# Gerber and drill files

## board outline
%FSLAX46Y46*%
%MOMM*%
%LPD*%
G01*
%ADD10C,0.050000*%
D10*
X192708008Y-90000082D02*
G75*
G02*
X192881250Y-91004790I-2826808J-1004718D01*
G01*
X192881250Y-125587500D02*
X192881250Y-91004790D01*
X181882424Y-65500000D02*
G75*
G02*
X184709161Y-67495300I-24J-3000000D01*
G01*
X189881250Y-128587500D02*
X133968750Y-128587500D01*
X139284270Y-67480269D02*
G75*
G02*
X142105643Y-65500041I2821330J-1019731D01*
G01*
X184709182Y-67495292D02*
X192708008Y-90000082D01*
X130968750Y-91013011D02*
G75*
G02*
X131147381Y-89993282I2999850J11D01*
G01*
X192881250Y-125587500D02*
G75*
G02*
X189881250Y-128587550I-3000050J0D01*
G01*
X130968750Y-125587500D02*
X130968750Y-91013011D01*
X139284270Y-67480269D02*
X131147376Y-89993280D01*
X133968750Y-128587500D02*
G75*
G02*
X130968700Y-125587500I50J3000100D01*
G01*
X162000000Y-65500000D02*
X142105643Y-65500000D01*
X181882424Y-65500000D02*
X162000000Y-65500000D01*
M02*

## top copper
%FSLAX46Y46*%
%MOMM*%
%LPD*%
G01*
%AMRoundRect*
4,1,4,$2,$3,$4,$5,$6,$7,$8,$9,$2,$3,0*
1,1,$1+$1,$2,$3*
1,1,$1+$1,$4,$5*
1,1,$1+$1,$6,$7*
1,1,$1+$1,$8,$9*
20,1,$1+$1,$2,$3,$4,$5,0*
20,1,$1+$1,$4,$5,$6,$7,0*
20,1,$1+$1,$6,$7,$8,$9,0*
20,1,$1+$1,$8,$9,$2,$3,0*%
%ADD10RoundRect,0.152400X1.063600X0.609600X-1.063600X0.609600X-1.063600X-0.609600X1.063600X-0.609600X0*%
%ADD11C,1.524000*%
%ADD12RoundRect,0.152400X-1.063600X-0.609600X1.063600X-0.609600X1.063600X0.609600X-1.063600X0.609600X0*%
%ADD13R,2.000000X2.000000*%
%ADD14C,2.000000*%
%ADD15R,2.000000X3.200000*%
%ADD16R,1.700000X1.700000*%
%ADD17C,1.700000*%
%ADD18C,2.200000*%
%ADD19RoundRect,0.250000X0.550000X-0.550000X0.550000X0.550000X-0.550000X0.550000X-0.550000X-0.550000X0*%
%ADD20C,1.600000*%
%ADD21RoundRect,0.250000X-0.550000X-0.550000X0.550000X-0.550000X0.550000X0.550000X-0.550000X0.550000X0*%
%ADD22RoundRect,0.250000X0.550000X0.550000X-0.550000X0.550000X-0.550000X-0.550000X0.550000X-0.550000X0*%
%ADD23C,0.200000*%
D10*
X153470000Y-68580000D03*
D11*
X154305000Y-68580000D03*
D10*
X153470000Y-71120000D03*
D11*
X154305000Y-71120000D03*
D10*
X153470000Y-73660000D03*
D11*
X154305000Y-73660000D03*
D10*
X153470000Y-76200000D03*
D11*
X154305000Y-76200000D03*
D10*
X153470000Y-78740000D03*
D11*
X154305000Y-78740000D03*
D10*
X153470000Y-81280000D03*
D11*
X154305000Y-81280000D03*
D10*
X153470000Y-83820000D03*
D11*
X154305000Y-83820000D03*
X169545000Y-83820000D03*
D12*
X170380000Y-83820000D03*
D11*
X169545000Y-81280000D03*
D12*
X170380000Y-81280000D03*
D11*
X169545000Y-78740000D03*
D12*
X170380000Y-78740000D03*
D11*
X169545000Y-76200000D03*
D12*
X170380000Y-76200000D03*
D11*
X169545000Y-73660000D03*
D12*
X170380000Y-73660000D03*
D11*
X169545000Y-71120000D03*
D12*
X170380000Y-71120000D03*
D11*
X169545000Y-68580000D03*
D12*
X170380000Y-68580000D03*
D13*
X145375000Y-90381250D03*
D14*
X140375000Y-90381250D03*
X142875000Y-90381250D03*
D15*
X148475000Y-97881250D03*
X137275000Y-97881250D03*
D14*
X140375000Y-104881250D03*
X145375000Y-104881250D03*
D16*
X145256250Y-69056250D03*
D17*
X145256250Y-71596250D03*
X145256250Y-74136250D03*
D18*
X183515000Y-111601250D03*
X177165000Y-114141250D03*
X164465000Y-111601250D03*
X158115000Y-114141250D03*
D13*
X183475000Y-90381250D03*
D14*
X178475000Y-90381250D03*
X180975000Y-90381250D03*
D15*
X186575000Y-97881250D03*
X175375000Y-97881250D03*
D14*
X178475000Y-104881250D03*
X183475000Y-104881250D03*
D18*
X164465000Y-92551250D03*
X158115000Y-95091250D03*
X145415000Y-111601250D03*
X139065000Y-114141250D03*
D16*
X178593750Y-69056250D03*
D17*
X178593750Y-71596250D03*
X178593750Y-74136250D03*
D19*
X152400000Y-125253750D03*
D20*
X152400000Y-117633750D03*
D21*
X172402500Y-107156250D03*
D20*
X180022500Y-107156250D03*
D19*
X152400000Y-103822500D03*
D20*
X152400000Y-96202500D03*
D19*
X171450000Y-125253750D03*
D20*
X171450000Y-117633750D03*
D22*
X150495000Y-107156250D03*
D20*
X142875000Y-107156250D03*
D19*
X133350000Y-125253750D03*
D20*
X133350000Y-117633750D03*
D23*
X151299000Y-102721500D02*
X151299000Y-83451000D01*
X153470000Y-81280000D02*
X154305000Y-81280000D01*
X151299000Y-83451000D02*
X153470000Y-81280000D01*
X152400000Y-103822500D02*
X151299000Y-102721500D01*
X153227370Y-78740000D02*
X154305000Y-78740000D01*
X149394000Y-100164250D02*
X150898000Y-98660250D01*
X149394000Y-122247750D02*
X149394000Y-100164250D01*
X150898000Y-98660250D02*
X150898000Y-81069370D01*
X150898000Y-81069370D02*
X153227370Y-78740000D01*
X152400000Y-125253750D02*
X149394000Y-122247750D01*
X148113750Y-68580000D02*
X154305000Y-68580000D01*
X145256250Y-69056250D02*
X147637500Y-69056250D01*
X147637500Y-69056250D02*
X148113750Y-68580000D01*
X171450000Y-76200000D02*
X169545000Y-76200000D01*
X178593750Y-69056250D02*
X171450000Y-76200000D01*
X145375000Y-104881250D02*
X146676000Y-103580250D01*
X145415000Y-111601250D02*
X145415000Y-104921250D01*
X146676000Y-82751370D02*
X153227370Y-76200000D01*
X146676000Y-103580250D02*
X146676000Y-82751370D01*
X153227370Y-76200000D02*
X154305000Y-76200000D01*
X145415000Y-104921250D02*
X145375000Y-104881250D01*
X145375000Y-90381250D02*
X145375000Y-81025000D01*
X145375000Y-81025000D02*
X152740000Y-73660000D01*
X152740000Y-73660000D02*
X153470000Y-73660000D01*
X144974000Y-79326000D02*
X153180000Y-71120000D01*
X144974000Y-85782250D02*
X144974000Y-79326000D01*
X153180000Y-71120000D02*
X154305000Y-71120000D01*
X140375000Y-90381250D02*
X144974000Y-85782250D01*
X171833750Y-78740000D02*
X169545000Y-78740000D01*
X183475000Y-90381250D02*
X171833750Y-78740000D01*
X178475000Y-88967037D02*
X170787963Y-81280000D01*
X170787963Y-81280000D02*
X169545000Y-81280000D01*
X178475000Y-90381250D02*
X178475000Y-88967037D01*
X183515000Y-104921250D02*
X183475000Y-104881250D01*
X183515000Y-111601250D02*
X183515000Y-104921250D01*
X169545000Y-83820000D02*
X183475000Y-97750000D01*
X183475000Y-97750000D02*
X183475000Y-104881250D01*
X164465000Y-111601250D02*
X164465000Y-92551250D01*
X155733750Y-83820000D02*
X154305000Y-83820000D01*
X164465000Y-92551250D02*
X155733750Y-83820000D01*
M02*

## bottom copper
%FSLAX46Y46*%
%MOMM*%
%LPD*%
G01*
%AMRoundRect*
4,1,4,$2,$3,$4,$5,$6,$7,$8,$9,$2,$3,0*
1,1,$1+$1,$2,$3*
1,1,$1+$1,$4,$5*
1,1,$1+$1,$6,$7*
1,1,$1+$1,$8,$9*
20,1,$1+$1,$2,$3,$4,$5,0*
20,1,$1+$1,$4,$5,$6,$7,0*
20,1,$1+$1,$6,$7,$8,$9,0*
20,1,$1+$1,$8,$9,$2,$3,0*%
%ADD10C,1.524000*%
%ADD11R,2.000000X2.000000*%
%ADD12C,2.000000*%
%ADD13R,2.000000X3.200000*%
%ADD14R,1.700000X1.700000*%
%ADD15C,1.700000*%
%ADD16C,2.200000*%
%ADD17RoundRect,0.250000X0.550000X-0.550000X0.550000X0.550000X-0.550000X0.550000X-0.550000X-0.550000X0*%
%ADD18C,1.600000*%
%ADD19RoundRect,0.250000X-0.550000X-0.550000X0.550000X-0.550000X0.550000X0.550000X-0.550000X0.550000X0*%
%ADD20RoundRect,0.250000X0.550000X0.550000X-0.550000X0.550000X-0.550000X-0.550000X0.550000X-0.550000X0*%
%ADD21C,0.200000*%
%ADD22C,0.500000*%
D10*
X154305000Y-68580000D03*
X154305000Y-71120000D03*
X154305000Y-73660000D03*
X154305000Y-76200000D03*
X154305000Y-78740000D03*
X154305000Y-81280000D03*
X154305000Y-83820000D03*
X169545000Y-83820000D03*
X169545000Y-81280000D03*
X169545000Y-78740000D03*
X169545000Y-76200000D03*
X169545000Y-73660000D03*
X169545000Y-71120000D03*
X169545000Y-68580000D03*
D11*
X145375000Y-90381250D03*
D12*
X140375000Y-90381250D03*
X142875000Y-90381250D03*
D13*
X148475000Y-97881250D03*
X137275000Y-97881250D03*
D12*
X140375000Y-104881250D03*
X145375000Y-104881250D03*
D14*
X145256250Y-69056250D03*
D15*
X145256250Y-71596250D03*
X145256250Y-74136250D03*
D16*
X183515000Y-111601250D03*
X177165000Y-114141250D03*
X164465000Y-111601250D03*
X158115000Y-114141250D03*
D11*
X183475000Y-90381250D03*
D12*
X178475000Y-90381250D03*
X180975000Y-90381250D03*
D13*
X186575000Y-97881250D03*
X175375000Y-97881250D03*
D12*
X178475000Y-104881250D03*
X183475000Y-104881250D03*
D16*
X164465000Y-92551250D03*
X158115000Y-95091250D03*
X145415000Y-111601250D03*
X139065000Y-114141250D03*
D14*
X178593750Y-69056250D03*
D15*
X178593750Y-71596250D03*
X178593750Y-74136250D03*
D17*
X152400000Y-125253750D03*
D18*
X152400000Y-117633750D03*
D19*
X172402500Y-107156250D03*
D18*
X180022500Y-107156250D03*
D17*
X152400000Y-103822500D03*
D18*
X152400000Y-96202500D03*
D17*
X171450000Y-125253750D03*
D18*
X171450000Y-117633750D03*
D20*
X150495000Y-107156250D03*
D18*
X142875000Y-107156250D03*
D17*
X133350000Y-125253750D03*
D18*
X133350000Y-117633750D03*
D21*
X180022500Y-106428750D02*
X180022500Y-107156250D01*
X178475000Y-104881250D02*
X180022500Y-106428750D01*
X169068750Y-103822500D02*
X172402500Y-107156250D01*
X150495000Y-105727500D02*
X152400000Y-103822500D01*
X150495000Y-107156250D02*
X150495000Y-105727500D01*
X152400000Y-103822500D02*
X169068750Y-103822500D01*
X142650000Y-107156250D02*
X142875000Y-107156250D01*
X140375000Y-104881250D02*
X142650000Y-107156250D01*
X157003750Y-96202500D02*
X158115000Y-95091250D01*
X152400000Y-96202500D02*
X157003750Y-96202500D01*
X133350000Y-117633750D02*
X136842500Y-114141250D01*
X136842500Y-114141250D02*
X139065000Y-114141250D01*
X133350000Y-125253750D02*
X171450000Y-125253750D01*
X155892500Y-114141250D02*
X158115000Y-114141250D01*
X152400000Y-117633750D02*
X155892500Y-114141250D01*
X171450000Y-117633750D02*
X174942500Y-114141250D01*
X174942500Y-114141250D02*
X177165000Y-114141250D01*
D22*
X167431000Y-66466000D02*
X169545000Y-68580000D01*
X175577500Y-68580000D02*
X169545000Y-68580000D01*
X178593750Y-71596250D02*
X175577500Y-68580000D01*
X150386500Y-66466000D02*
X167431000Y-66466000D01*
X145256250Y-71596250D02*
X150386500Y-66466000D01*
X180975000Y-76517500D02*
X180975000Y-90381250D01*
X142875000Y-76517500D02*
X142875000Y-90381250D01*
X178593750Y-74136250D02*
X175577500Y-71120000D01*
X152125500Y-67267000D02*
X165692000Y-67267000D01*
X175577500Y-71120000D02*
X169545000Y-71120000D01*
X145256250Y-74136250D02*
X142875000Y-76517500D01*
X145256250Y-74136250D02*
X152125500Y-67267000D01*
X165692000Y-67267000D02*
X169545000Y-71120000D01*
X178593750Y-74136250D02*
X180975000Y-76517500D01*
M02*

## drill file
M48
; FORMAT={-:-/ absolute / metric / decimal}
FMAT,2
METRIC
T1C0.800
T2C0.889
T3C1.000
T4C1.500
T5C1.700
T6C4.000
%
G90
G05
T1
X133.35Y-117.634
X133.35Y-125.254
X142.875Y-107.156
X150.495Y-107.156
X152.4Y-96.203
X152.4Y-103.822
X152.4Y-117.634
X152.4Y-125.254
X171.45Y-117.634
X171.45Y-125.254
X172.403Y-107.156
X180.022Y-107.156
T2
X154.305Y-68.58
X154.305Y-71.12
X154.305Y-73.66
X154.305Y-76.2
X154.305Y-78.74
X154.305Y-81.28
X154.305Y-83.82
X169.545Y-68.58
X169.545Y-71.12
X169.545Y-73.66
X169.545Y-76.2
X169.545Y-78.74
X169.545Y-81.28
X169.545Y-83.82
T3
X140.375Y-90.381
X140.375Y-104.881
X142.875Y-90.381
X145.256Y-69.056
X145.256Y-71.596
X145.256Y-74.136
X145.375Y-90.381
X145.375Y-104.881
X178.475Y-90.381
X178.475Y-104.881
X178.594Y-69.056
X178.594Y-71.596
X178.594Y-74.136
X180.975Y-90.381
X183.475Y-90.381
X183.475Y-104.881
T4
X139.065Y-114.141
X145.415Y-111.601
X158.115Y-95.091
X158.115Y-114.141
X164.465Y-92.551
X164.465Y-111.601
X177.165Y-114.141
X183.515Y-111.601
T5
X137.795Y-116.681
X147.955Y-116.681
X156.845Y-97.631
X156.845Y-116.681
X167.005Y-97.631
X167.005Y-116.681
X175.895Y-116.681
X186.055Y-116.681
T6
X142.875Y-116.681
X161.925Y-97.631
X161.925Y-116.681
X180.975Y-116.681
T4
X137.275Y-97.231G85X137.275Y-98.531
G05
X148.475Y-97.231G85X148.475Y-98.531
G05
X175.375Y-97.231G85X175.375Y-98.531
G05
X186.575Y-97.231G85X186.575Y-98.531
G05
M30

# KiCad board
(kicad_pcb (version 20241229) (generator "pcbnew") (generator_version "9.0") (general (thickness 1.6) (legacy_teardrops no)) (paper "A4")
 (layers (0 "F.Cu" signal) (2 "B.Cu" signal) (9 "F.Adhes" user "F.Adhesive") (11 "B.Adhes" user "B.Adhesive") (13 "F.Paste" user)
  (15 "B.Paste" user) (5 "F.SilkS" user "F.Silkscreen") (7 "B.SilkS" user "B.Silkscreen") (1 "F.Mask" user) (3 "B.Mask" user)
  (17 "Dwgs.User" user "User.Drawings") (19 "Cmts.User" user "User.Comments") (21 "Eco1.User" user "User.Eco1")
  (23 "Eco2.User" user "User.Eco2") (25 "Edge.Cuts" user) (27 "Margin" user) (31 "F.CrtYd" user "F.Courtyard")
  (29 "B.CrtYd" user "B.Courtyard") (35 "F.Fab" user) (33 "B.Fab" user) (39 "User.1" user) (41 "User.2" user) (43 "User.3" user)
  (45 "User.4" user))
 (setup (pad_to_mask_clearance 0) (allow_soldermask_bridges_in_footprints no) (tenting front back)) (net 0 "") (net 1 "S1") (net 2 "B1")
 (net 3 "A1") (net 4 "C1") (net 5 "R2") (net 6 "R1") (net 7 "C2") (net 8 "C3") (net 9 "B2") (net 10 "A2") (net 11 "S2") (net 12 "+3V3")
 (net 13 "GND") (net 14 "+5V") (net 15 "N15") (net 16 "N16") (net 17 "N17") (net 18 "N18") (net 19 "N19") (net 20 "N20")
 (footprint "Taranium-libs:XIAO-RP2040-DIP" (layer "F.Cu") (at 161.925 76.2)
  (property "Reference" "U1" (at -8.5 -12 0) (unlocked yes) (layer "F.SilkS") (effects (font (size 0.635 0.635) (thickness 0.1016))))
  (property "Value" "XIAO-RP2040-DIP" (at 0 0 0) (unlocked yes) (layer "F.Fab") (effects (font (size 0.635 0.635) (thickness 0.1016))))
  (pad "1" smd roundrect (at -8.455 -7.62 180) (size 2.432 1.524) (layers "F.Cu" "F.Mask") (roundrect_rratio 0.1) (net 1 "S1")
   (thermal_bridge_angle 45))
  (pad "1" thru_hole circle (at -7.62 -7.62 180) (size 1.524 1.524) (drill 0.889) (layers "*.Cu" "*.Mask") (remove_unused_layers no)
   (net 1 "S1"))
  (pad "2" smd roundrect (at -8.455 -5.08 180) (size 2.432 1.524) (layers "F.Cu" "F.Mask") (roundrect_rratio 0.1) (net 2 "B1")
   (thermal_bridge_angle 45))
  (pad "2" thru_hole circle (at -7.62 -5.08 180) (size 1.524 1.524) (drill 0.889) (layers "*.Cu" "*.Mask") (remove_unused_layers no)
   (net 2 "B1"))
  (pad "3" smd roundrect (at -8.455 -2.54 180) (size 2.432 1.524) (layers "F.Cu" "F.Mask") (roundrect_rratio 0.1) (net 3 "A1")
   (thermal_bridge_angle 45))
  (pad "3" thru_hole circle (at -7.62 -2.54 180) (size 1.524 1.524) (drill 0.889) (layers "*.Cu" "*.Mask") (remove_unused_layers no)
   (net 3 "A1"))
  (pad "4" smd roundrect (at -8.455 0 180) (size 2.432 1.524) (layers "F.Cu" "F.Mask") (roundrect_rratio 0.1) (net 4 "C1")
   (thermal_bridge_angle 45))
  (pad "4" thru_hole circle (at -7.62 0 180) (size 1.524 1.524) (drill 0.889) (layers "*.Cu" "*.Mask") (remove_unused_layers no)
   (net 4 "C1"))
  (pad "5" smd roundrect (at -8.455 2.54 180) (size 2.432 1.524) (layers "F.Cu" "F.Mask") (roundrect_rratio 0.1) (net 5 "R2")
   (thermal_bridge_angle 45))
  (pad "5" thru_hole circle (at -7.62 2.54 180) (size 1.524 1.524) (drill 0.889) (layers "*.Cu" "*.Mask") (remove_unused_layers no)
   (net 5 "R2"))
  (pad "6" smd roundrect (at -8.455 5.08 180) (size 2.432 1.524) (layers "F.Cu" "F.Mask") (roundrect_rratio 0.1) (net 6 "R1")
   (thermal_bridge_angle 45))
  (pad "6" thru_hole circle (at -7.62 5.08 180) (size 1.524 1.524) (drill 0.889) (layers "*.Cu" "*.Mask") (remove_unused_layers no)
   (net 6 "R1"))
  (pad "7" smd roundrect (at -8.455 7.62 180) (size 2.432 1.524) (layers "F.Cu" "F.Mask") (roundrect_rratio 0.1) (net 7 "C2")
   (thermal_bridge_angle 45))
  (pad "7" thru_hole circle (at -7.62 7.62 180) (size 1.524 1.524) (drill 0.889) (layers "*.Cu" "*.Mask") (remove_unused_layers no)
   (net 7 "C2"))
  (pad "8" thru_hole circle (at 7.62 7.62) (size 1.524 1.524) (drill 0.889) (layers "*.Cu" "*.Mask") (remove_unused_layers no) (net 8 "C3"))
  (pad "8" smd roundrect (at 8.455 7.62) (size 2.432 1.524) (layers "F.Cu" "F.Mask") (roundrect_rratio 0.1) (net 8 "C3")
   (thermal_bridge_angle 45))
  (pad "9" thru_hole circle (at 7.62 5.08) (size 1.524 1.524) (drill 0.889) (layers "*.Cu" "*.Mask") (remove_unused_layers no) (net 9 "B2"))
  (pad "9" smd roundrect (at 8.455 5.08) (size 2.432 1.524) (layers "F.Cu" "F.Mask") (roundrect_rratio 0.1) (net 9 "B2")
   (thermal_bridge_angle 45))
  (pad "10" thru_hole circle (at 7.62 2.54) (size 1.524 1.524) (drill 0.889) (layers "*.Cu" "*.Mask") (remove_unused_layers no)
   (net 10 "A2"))
  (pad "10" smd roundrect (at 8.455 2.54) (size 2.432 1.524) (layers "F.Cu" "F.Mask") (roundrect_rratio 0.1) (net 10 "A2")
   (thermal_bridge_angle 45))
  (pad "11" thru_hole circle (at 7.62 0) (size 1.524 1.524) (drill 0.889) (layers "*.Cu" "*.Mask") (remove_unused_layers no) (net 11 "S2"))
  (pad "11" smd roundrect (at 8.455 0) (size 2.432 1.524) (layers "F.Cu" "F.Mask") (roundrect_rratio 0.1) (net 11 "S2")
   (thermal_bridge_angle 45))
  (pad "12" thru_hole circle (at 7.62 -2.54) (size 1.524 1.524) (drill 0.889) (layers "*.Cu" "*.Mask") (remove_unused_layers no)
   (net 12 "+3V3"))
  (pad "12" smd roundrect (at 8.455 -2.54) (size 2.432 1.524) (layers "F.Cu" "F.Mask") (roundrect_rratio 0.1) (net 12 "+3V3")
   (thermal_bridge_angle 45))
  (pad "13" thru_hole circle (at 7.62 -5.08) (size 1.524 1.524) (drill 0.889) (layers "*.Cu" "*.Mask") (remove_unused_layers no)
   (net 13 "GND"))
  (pad "13" smd roundrect (at 8.455 -5.08) (size 2.432 1.524) (layers "F.Cu" "F.Mask") (roundrect_rratio 0.1) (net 13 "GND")
   (thermal_bridge_angle 45))
  (pad "14" thru_hole circle (at 7.62 -7.62) (size 1.524 1.524) (drill 0.889) (layers "*.Cu" "*.Mask") (remove_unused_layers no)
   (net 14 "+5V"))
  (pad "14" smd roundrect (at 8.455 -7.62) (size 2.432 1.524) (layers "F.Cu" "F.Mask") (roundrect_rratio 0.1) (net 14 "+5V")
   (thermal_bridge_angle 45)))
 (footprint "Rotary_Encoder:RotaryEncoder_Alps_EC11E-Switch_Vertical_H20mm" (layer "F.Cu") (at 145.375 90.38125 -90)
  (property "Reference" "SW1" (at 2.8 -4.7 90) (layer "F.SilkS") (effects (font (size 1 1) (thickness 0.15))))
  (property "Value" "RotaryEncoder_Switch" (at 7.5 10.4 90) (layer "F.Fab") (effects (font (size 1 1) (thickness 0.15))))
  (pad "A" thru_hole rect (at 0 0 270) (size 2 2) (drill 1) (layers "*.Cu" "*.Mask") (remove_unused_layers no) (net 3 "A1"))
  (pad "B" thru_hole circle (at 0 5 270) (size 2 2) (drill 1) (layers "*.Cu" "*.Mask") (remove_unused_layers no) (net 2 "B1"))
  (pad "C" thru_hole circle (at 0 2.5 270) (size 2 2) (drill 1) (layers "*.Cu" "*.Mask") (remove_unused_layers no) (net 13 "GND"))
  (pad "MP" thru_hole rect (at 7.5 -3.1 270) (size 3.2 2) (drill oval 2.8 1.5) (layers "*.Cu" "*.Mask") (remove_unused_layers no))
  (pad "MP" thru_hole rect (at 7.5 8.1 270) (size 3.2 2) (drill oval 2.8 1.5) (layers "*.Cu" "*.Mask") (remove_unused_layers no))
  (pad "S1" thru_hole circle (at 14.5 5 270) (size 2 2) (drill 1) (layers "*.Cu" "*.Mask") (remove_unused_layers no) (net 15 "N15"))
  (pad "S2" thru_hole circle (at 14.5 0 270) (size 2 2) (drill 1) (layers "*.Cu" "*.Mask") (remove_unused_layers no) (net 4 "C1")))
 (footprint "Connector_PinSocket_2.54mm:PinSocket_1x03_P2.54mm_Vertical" (layer "F.Cu") (at 145.25625 69.05625)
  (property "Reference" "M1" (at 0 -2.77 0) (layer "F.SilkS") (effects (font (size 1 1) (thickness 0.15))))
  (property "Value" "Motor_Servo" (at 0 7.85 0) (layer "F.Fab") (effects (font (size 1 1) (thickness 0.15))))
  (pad "1" thru_hole rect (at 0 0) (size 1.7 1.7) (drill 1) (layers "*.Cu" "*.Mask") (remove_unused_layers no) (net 1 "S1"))
  (pad "2" thru_hole circle (at 0 2.54) (size 1.7 1.7) (drill 1) (layers "*.Cu" "*.Mask") (remove_unused_layers no) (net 14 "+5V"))
  (pad "3" thru_hole circle (at 0 5.08) (size 1.7 1.7) (drill 1) (layers "*.Cu" "*.Mask") (remove_unused_layers no) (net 13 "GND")))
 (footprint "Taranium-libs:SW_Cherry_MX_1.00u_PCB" (layer "F.Cu") (at 183.515 111.60125)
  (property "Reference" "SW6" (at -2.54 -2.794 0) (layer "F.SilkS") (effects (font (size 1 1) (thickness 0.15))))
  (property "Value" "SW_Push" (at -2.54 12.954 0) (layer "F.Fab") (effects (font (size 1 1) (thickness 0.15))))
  (pad "" np_thru_hole circle (at -7.62 5.08) (size 1.7 1.7) (drill 1.7) (layers "*.Cu" "*.Mask"))
  (pad "" np_thru_hole circle (at -2.54 5.08) (size 4 4) (drill 4) (layers "*.Cu" "*.Mask"))
  (pad "" np_thru_hole circle (at 2.54 5.08) (size 1.7 1.7) (drill 1.7) (layers "*.Cu" "*.Mask"))
  (pad "1" thru_hole circle (at 0 0) (size 2.2 2.2) (drill 1.5) (layers "*.Cu" "*.Mask") (remove_unused_layers no) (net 8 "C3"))
  (pad "2" thru_hole circle (at -6.35 2.54) (size 2.2 2.2) (drill 1.5) (layers "*.Cu" "*.Mask") (remove_unused_layers no) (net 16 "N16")))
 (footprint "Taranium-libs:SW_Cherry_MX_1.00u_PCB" (layer "F.Cu") (at 164.465 111.60125)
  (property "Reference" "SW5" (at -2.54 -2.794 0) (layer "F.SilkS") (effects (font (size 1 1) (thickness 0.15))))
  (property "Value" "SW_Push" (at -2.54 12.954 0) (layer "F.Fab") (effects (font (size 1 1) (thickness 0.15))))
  (pad "" np_thru_hole circle (at -7.62 5.08) (size 1.7 1.7) (drill 1.7) (layers "*.Cu" "*.Mask"))
  (pad "" np_thru_hole circle (at -2.54 5.08) (size 4 4) (drill 4) (layers "*.Cu" "*.Mask"))
  (pad "" np_thru_hole circle (at 2.54 5.08) (size 1.7 1.7) (drill 1.7) (layers "*.Cu" "*.Mask"))
  (pad "1" thru_hole circle (at 0 0) (size 2.2 2.2) (drill 1.5) (layers "*.Cu" "*.Mask") (remove_unused_layers no) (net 7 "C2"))
  (pad "2" thru_hole circle (at -6.35 2.54) (size 2.2 2.2) (drill 1.5) (layers "*.Cu" "*.Mask") (remove_unused_layers no) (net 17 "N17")))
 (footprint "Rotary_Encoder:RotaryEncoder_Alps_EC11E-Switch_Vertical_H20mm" (layer "F.Cu") (at 183.475 90.38125 -90)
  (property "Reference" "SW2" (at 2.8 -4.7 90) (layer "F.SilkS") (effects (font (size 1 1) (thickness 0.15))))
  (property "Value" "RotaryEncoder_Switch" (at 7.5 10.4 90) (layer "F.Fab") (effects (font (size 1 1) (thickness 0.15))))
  (pad "A" thru_hole rect (at 0 0 270) (size 2 2) (drill 1) (layers "*.Cu" "*.Mask") (remove_unused_layers no) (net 10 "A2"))
  (pad "B" thru_hole circle (at 0 5 270) (size 2 2) (drill 1) (layers "*.Cu" "*.Mask") (remove_unused_layers no) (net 9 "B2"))
  (pad "C" thru_hole circle (at 0 2.5 270) (size 2 2) (drill 1) (layers "*.Cu" "*.Mask") (remove_unused_layers no) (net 13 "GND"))
  (pad "MP" thru_hole rect (at 7.5 -3.1 270) (size 3.2 2) (drill oval 2.8 1.5) (layers "*.Cu" "*.Mask") (remove_unused_layers no))
  (pad "MP" thru_hole rect (at 7.5 8.1 270) (size 3.2 2) (drill oval 2.8 1.5) (layers "*.Cu" "*.Mask") (remove_unused_layers no))
  (pad "S1" thru_hole circle (at 14.5 5 270) (size 2 2) (drill 1) (layers "*.Cu" "*.Mask") (remove_unused_layers no) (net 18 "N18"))
  (pad "S2" thru_hole circle (at 14.5 0 270) (size 2 2) (drill 1) (layers "*.Cu" "*.Mask") (remove_unused_layers no) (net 8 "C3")))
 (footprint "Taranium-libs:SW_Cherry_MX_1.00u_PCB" (layer "F.Cu") (at 164.465 92.55125)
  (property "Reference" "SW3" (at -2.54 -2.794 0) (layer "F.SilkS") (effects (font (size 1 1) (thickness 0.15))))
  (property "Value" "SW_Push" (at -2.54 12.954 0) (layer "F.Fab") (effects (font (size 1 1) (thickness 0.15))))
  (pad "" np_thru_hole circle (at -7.62 5.08) (size 1.7 1.7) (drill 1.7) (layers "*.Cu" "*.Mask"))
  (pad "" np_thru_hole circle (at -2.54 5.08) (size 4 4) (drill 4) (layers "*.Cu" "*.Mask"))
  (pad "" np_thru_hole circle (at 2.54 5.08) (size 1.7 1.7) (drill 1.7) (layers "*.Cu" "*.Mask"))
  (pad "1" thru_hole circle (at 0 0) (size 2.2 2.2) (drill 1.5) (layers "*.Cu" "*.Mask") (remove_unused_layers no) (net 7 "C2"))
  (pad "2" thru_hole circle (at -6.35 2.54) (size 2.2 2.2) (drill 1.5) (layers "*.Cu" "*.Mask") (remove_unused_layers no) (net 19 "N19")))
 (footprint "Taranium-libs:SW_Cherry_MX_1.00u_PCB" (layer "F.Cu") (at 145.415 111.60125)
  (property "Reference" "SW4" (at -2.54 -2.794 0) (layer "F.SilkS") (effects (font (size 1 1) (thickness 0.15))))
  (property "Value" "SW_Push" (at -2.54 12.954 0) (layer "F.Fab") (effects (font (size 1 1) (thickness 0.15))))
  (pad "" np_thru_hole circle (at -7.62 5.08) (size 1.7 1.7) (drill 1.7) (layers "*.Cu" "*.Mask"))
  (pad "" np_thru_hole circle (at -2.54 5.08) (size 4 4) (drill 4) (layers "*.Cu" "*.Mask"))
  (pad "" np_thru_hole circle (at 2.54 5.08) (size 1.7 1.7) (drill 1.7) (layers "*.Cu" "*.Mask"))
  (pad "1" thru_hole circle (at 0 0) (size 2.2 2.2) (drill 1.5) (layers "*.Cu" "*.Mask") (remove_unused_layers no) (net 4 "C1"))
  (pad "2" thru_hole circle (at -6.35 2.54) (size 2.2 2.2) (drill 1.5) (layers "*.Cu" "*.Mask") (remove_unused_layers no) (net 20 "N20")))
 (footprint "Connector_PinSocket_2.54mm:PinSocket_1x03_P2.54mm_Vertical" (layer "F.Cu") (at 178.59375 69.05625)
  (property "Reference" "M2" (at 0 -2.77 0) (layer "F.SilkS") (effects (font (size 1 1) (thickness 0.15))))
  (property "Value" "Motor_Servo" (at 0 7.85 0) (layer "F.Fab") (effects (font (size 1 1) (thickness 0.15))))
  (pad "1" thru_hole rect (at 0 0) (size 1.7 1.7) (drill 1) (layers "*.Cu" "*.Mask") (remove_unused_layers no) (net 11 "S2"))
  (pad "2" thru_hole circle (at 0 2.54) (size 1.7 1.7) (drill 1) (layers "*.Cu" "*.Mask") (remove_unused_layers no) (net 14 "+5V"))
  (pad "3" thru_hole circle (at 0 5.08) (size 1.7 1.7) (drill 1) (layers "*.Cu" "*.Mask") (remove_unused_layers no) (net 13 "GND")))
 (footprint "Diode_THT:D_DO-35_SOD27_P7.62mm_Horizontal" (layer "B.Cu") (at 152.4 125.25375 90)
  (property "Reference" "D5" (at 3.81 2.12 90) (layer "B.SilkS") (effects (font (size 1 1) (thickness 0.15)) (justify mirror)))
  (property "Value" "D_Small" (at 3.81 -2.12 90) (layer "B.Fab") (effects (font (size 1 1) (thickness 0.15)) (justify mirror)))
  (pad "1" thru_hole roundrect (at 0 0 90) (size 1.6 1.6) (drill 0.8) (layers "*.Cu" "*.Mask") (remove_unused_layers no)
   (roundrect_rratio 0.15625) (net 5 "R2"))
  (pad "2" thru_hole circle (at 7.62 0 90) (size 1.6 1.6) (drill 0.8) (layers "*.Cu" "*.Mask") (remove_unused_layers no) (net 17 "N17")))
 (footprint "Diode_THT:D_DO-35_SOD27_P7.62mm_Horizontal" (layer "B.Cu") (at 172.4025 107.15625)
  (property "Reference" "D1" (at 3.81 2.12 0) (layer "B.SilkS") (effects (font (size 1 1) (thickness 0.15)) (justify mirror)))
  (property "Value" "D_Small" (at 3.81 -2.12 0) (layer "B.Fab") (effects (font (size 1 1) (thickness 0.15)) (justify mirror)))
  (pad "1" thru_hole roundrect (at 0 0) (size 1.6 1.6) (drill 0.8) (layers "*.Cu" "*.Mask") (remove_unused_layers no)
   (roundrect_rratio 0.15625) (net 6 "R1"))
  (pad "2" thru_hole circle (at 7.62 0) (size 1.6 1.6) (drill 0.8) (layers "*.Cu" "*.Mask") (remove_unused_layers no) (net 18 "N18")))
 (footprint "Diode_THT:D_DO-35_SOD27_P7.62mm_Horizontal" (layer "B.Cu") (at 152.4 103.8225 90)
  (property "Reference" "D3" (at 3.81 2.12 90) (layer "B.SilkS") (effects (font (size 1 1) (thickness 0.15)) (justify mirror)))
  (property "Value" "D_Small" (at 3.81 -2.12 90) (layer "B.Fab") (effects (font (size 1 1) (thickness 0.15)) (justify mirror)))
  (pad "1" thru_hole roundrect (at 0 0 90) (size 1.6 1.6) (drill 0.8) (layers "*.Cu" "*.Mask") (remove_unused_layers no)
   (roundrect_rratio 0.15625) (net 6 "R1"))
  (pad "2" thru_hole circle (at 7.62 0 90) (size 1.6 1.6) (drill 0.8) (layers "*.Cu" "*.Mask") (remove_unused_layers no) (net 19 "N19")))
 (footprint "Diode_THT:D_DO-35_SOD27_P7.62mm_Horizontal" (layer "B.Cu") (at 171.45 125.25375 90)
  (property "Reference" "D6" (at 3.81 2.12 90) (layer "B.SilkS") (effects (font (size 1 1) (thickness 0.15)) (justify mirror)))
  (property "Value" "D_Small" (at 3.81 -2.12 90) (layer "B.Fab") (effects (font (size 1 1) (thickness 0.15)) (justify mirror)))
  (pad "1" thru_hole roundrect (at 0 0 90) (size 1.6 1.6) (drill 0.8) (layers "*.Cu" "*.Mask") (remove_unused_layers no)
   (roundrect_rratio 0.15625) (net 5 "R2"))
  (pad "2" thru_hole circle (at 7.62 0 90) (size 1.6 1.6) (drill 0.8) (layers "*.Cu" "*.Mask") (remove_unused_layers no) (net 16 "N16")))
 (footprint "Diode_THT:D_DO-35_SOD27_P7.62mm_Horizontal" (layer "B.Cu") (at 150.495 107.15625 180)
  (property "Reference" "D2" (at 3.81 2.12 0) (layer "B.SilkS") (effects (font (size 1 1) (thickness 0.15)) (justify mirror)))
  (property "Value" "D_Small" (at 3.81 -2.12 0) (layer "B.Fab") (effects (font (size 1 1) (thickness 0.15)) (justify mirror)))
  (pad "1" thru_hole roundrect (at 0 0 180) (size 1.6 1.6) (drill 0.8) (layers "*.Cu" "*.Mask") (remove_unused_layers no)
   (roundrect_rratio 0.15625) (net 6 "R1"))
  (pad "2" thru_hole circle (at 7.62 0 180) (size 1.6 1.6) (drill 0.8) (layers "*.Cu" "*.Mask") (remove_unused_layers no) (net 15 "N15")))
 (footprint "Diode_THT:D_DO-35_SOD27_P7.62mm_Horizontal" (layer "B.Cu") (at 133.35 125.25375 90)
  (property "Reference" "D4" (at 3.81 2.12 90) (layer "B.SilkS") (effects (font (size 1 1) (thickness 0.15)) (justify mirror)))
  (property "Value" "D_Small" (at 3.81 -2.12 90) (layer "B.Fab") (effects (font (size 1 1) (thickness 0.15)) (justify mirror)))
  (pad "1" thru_hole roundrect (at 0 0 90) (size 1.6 1.6) (drill 0.8) (layers "*.Cu" "*.Mask") (remove_unused_layers no)
   (roundrect_rratio 0.15625) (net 5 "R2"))
  (pad "2" thru_hole circle (at 7.62 0 90) (size 1.6 1.6) (drill 0.8) (layers "*.Cu" "*.Mask") (remove_unused_layers no) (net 20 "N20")))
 (gr_arc (start 192.708008 90.000082) (mid 192.837622 90.495023) (end 192.88125 91.00479) (stroke (width 0.05) (type default))
  (layer "Edge.Cuts"))
 (gr_line (start 192.88125 125.5875) (end 192.88125 91.00479) (stroke (width 0.05) (type default)) (layer "Edge.Cuts"))
 (gr_arc (start 181.882424 65.5) (mid 183.612435 66.049069) (end 184.709182 67.495292) (stroke (width 0.05) (type default))
  (layer "Edge.Cuts"))
 (gr_line (start 189.88125 128.5875) (end 133.96875 128.5875) (stroke (width 0.05) (type default)) (layer "Edge.Cuts"))
 (gr_arc (start 139.28427 67.480269) (mid 140.382158 66.044477) (end 142.105643 65.5) (stroke (width 0.05) (type default))
  (layer "Edge.Cuts"))
 (gr_line (start 184.709182 67.495292) (end 192.708008 90.000082) (stroke (width 0.05) (type default)) (layer "Edge.Cuts"))
 (gr_arc (start 130.96875 91.013011) (mid 131.013741 90.495381) (end 131.147376 89.99328) (stroke (width 0.05) (type default))
  (layer "Edge.Cuts"))
 (gr_arc (start 192.88125 125.5875) (mid 192.00257 127.70882) (end 189.88125 128.5875) (stroke (width 0.05) (type default))
  (layer "Edge.Cuts"))
 (gr_line (start 130.96875 125.5875) (end 130.96875 91.013011) (stroke (width 0.05) (type default)) (layer "Edge.Cuts"))
 (gr_line (start 139.28427 67.480269) (end 131.147376 89.99328) (stroke (width 0.05) (type default)) (layer "Edge.Cuts"))
 (gr_arc (start 133.96875 128.5875) (mid 131.847462 127.708803) (end 130.96875 125.5875) (stroke (width 0.05) (type default))
  (layer "Edge.Cuts"))
 (gr_line (start 162 65.5) (end 142.105643 65.5) (stroke (width 0.05) (type default)) (layer "Edge.Cuts"))
 (gr_line (start 181.882424 65.5) (end 162 65.5) (stroke (width 0.05) (type default)) (layer "Edge.Cuts"))
 (segment (start 180.0225 106.42875) (end 180.0225 107.15625) (width 0.2) (layer "B.Cu") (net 18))
 (segment (start 178.475 104.88125) (end 180.0225 106.42875) (width 0.2) (layer "B.Cu") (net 18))
 (segment (start 151.299 102.7215) (end 151.299 83.451) (width 0.2) (layer "F.Cu") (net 6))
 (segment (start 153.47 81.28) (end 154.305 81.28) (width 0.2) (layer "F.Cu") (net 6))
 (segment (start 151.299 83.451) (end 153.47 81.28) (width 0.2) (layer "F.Cu") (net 6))
 (segment (start 152.4 103.8225) (end 151.299 102.7215) (width 0.2) (layer "F.Cu") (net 6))
 (segment (start 169.06875 103.8225) (end 172.4025 107.15625) (width 0.2) (layer "B.Cu") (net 6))
 (segment (start 150.495 105.7275) (end 152.4 103.8225) (width 0.2) (layer "B.Cu") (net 6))
 (segment (start 150.495 107.15625) (end 150.495 105.7275) (width 0.2) (layer "B.Cu") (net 6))
 (segment (start 152.4 103.8225) (end 169.06875 103.8225) (width 0.2) (layer "B.Cu") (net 6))
 (segment (start 142.65 107.15625) (end 142.875 107.15625) (width 0.2) (layer "B.Cu") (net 15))
 (segment (start 140.375 104.88125) (end 142.65 107.15625) (width 0.2) (layer "B.Cu") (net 15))
 (segment (start 157.00375 96.2025) (end 158.115 95.09125) (width 0.2) (layer "B.Cu") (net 19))
 (segment (start 152.4 96.2025) (end 157.00375 96.2025) (width 0.2) (layer "B.Cu") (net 19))
 (segment (start 133.35 117.63375) (end 136.8425 114.14125) (width 0.2) (layer "B.Cu") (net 20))
 (segment (start 136.8425 114.14125) (end 139.065 114.14125) (width 0.2) (layer "B.Cu") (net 20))
 (segment (start 153.22737 78.74) (end 154.305 78.74) (width 0.2) (layer "F.Cu") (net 5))
 (segment (start 149.394 100.16425) (end 150.898 98.66025) (width 0.2) (layer "F.Cu") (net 5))
 (segment (start 149.394 122.24775) (end 149.394 100.16425) (width 0.2) (layer "F.Cu") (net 5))
 (segment (start 150.898 98.66025) (end 150.898 81.06937) (width 0.2) (layer "F.Cu") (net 5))
 (segment (start 150.898 81.06937) (end 153.22737 78.74) (width 0.2) (layer "F.Cu") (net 5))
 (segment (start 152.4 125.25375) (end 149.394 122.24775) (width 0.2) (layer "F.Cu") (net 5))
 (segment (start 133.35 125.25375) (end 171.45 125.25375) (width 0.2) (layer "B.Cu") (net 5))
 (segment (start 155.8925 114.14125) (end 158.115 114.14125) (width 0.2) (layer "B.Cu") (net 17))
 (segment (start 152.4 117.63375) (end 155.8925 114.14125) (width 0.2) (layer "B.Cu") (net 17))
 (segment (start 171.45 117.63375) (end 174.9425 114.14125) (width 0.2) (layer "B.Cu") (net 16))
 (segment (start 174.9425 114.14125) (end 177.165 114.14125) (width 0.2) (layer "B.Cu") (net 16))
 (segment (start 167.431 66.466) (end 169.545 68.58) (width 0.5) (layer "B.Cu") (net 14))
 (segment (start 175.5775 68.58) (end 169.545 68.58) (width 0.5) (layer "B.Cu") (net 14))
 (segment (start 178.59375 71.59625) (end 175.5775 68.58) (width 0.5) (layer "B.Cu") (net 14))
 (segment (start 150.3865 66.466) (end 167.431 66.466) (width 0.5) (layer "B.Cu") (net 14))
 (segment (start 145.25625 71.59625) (end 150.3865 66.466) (width 0.5) (layer "B.Cu") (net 14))
 (segment (start 180.975 76.5175) (end 180.975 90.38125) (width 0.5) (layer "B.Cu") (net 13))
 (segment (start 142.875 76.5175) (end 142.875 90.38125) (width 0.5) (layer "B.Cu") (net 13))
 (segment (start 178.59375 74.13625) (end 175.5775 71.12) (width 0.5) (layer "B.Cu") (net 13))
 (segment (start 152.1255 67.267) (end 165.692 67.267) (width 0.5) (layer "B.Cu") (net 13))
 (segment (start 175.5775 71.12) (end 169.545 71.12) (width 0.5) (layer "B.Cu") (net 13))
 (segment (start 145.25625 74.13625) (end 142.875 76.5175) (width 0.5) (layer "B.Cu") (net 13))
 (segment (start 145.25625 74.13625) (end 152.1255 67.267) (width 0.5) (layer "B.Cu") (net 13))
 (segment (start 165.692 67.267) (end 169.545 71.12) (width 0.5) (layer "B.Cu") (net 13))
 (segment (start 178.59375 74.13625) (end 180.975 76.5175) (width 0.5) (layer "B.Cu") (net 13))
 (segment (start 148.11375 68.58) (end 154.305 68.58) (width 0.2) (layer "F.Cu") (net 1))
 (segment (start 145.25625 69.05625) (end 147.6375 69.05625) (width 0.2) (layer "F.Cu") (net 1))
 (segment (start 147.6375 69.05625) (end 148.11375 68.58) (width 0.2) (layer "F.Cu") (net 1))
 (segment (start 171.45 76.2) (end 169.545 76.2) (width 0.2) (layer "F.Cu") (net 11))
 (segment (start 178.59375 69.05625) (end 171.45 76.2) (width 0.2) (layer "F.Cu") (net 11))
 (segment (start 145.375 104.88125) (end 146.676 103.58025) (width 0.2) (layer "F.Cu") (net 4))
 (segment (start 145.415 111.60125) (end 145.415 104.92125) (width 0.2) (layer "F.Cu") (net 4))
 (segment (start 146.676 82.75137) (end 153.22737 76.2) (width 0.2) (layer "F.Cu") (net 4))
 (segment (start 146.676 103.58025) (end 146.676 82.75137) (width 0.2) (layer "F.Cu") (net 4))
 (segment (start 153.22737 76.2) (end 154.305 76.2) (width 0.2) (layer "F.Cu") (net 4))
 (segment (start 145.415 104.92125) (end 145.375 104.88125) (width 0.2) (layer "F.Cu") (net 4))
 (segment (start 145.375 90.38125) (end 145.375 81.025) (width 0.2) (layer "F.Cu") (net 3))
 (segment (start 145.375 81.025) (end 152.74 73.66) (width 0.2) (layer "F.Cu") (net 3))
 (segment (start 152.74 73.66) (end 153.47 73.66) (width 0.2) (layer "F.Cu") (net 3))
 (segment (start 144.974 79.326) (end 153.18 71.12) (width 0.2) (layer "F.Cu") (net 2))
 (segment (start 144.974 85.78225) (end 144.974 79.326) (width 0.2) (layer "F.Cu") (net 2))
 (segment (start 153.18 71.12) (end 154.305 71.12) (width 0.2) (layer "F.Cu") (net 2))
 (segment (start 140.375 90.38125) (end 144.974 85.78225) (width 0.2) (layer "F.Cu") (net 2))
 (segment (start 171.83375 78.74) (end 169.545 78.74) (width 0.2) (layer "F.Cu") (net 10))
 (segment (start 183.475 90.38125) (end 171.83375 78.74) (width 0.2) (layer "F.Cu") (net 10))
 (segment (start 178.475 88.967037) (end 170.787963 81.28) (width 0.2) (layer "F.Cu") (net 9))
 (segment (start 170.787963 81.28) (end 169.545 81.28) (width 0.2) (layer "F.Cu") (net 9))
 (segment (start 178.475 90.38125) (end 178.475 88.967037) (width 0.2) (layer "F.Cu") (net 9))
 (segment (start 183.515 104.92125) (end 183.475 104.88125) (width 0.2) (layer "F.Cu") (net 8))
 (segment (start 183.515 111.60125) (end 183.515 104.92125) (width 0.2) (layer "F.Cu") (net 8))
 (segment (start 169.545 83.82) (end 183.475 97.75) (width 0.2) (layer "F.Cu") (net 8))
 (segment (start 183.475 97.75) (end 183.475 104.88125) (width 0.2) (layer "F.Cu") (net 8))
 (segment (start 164.465 111.60125) (end 164.465 92.55125) (width 0.2) (layer "F.Cu") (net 7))
 (segment (start 155.73375 83.82) (end 154.305 83.82) (width 0.2) (layer "F.Cu") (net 7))
 (segment (start 164.465 92.55125) (end 155.73375 83.82) (width 0.2) (layer "F.Cu") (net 7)))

